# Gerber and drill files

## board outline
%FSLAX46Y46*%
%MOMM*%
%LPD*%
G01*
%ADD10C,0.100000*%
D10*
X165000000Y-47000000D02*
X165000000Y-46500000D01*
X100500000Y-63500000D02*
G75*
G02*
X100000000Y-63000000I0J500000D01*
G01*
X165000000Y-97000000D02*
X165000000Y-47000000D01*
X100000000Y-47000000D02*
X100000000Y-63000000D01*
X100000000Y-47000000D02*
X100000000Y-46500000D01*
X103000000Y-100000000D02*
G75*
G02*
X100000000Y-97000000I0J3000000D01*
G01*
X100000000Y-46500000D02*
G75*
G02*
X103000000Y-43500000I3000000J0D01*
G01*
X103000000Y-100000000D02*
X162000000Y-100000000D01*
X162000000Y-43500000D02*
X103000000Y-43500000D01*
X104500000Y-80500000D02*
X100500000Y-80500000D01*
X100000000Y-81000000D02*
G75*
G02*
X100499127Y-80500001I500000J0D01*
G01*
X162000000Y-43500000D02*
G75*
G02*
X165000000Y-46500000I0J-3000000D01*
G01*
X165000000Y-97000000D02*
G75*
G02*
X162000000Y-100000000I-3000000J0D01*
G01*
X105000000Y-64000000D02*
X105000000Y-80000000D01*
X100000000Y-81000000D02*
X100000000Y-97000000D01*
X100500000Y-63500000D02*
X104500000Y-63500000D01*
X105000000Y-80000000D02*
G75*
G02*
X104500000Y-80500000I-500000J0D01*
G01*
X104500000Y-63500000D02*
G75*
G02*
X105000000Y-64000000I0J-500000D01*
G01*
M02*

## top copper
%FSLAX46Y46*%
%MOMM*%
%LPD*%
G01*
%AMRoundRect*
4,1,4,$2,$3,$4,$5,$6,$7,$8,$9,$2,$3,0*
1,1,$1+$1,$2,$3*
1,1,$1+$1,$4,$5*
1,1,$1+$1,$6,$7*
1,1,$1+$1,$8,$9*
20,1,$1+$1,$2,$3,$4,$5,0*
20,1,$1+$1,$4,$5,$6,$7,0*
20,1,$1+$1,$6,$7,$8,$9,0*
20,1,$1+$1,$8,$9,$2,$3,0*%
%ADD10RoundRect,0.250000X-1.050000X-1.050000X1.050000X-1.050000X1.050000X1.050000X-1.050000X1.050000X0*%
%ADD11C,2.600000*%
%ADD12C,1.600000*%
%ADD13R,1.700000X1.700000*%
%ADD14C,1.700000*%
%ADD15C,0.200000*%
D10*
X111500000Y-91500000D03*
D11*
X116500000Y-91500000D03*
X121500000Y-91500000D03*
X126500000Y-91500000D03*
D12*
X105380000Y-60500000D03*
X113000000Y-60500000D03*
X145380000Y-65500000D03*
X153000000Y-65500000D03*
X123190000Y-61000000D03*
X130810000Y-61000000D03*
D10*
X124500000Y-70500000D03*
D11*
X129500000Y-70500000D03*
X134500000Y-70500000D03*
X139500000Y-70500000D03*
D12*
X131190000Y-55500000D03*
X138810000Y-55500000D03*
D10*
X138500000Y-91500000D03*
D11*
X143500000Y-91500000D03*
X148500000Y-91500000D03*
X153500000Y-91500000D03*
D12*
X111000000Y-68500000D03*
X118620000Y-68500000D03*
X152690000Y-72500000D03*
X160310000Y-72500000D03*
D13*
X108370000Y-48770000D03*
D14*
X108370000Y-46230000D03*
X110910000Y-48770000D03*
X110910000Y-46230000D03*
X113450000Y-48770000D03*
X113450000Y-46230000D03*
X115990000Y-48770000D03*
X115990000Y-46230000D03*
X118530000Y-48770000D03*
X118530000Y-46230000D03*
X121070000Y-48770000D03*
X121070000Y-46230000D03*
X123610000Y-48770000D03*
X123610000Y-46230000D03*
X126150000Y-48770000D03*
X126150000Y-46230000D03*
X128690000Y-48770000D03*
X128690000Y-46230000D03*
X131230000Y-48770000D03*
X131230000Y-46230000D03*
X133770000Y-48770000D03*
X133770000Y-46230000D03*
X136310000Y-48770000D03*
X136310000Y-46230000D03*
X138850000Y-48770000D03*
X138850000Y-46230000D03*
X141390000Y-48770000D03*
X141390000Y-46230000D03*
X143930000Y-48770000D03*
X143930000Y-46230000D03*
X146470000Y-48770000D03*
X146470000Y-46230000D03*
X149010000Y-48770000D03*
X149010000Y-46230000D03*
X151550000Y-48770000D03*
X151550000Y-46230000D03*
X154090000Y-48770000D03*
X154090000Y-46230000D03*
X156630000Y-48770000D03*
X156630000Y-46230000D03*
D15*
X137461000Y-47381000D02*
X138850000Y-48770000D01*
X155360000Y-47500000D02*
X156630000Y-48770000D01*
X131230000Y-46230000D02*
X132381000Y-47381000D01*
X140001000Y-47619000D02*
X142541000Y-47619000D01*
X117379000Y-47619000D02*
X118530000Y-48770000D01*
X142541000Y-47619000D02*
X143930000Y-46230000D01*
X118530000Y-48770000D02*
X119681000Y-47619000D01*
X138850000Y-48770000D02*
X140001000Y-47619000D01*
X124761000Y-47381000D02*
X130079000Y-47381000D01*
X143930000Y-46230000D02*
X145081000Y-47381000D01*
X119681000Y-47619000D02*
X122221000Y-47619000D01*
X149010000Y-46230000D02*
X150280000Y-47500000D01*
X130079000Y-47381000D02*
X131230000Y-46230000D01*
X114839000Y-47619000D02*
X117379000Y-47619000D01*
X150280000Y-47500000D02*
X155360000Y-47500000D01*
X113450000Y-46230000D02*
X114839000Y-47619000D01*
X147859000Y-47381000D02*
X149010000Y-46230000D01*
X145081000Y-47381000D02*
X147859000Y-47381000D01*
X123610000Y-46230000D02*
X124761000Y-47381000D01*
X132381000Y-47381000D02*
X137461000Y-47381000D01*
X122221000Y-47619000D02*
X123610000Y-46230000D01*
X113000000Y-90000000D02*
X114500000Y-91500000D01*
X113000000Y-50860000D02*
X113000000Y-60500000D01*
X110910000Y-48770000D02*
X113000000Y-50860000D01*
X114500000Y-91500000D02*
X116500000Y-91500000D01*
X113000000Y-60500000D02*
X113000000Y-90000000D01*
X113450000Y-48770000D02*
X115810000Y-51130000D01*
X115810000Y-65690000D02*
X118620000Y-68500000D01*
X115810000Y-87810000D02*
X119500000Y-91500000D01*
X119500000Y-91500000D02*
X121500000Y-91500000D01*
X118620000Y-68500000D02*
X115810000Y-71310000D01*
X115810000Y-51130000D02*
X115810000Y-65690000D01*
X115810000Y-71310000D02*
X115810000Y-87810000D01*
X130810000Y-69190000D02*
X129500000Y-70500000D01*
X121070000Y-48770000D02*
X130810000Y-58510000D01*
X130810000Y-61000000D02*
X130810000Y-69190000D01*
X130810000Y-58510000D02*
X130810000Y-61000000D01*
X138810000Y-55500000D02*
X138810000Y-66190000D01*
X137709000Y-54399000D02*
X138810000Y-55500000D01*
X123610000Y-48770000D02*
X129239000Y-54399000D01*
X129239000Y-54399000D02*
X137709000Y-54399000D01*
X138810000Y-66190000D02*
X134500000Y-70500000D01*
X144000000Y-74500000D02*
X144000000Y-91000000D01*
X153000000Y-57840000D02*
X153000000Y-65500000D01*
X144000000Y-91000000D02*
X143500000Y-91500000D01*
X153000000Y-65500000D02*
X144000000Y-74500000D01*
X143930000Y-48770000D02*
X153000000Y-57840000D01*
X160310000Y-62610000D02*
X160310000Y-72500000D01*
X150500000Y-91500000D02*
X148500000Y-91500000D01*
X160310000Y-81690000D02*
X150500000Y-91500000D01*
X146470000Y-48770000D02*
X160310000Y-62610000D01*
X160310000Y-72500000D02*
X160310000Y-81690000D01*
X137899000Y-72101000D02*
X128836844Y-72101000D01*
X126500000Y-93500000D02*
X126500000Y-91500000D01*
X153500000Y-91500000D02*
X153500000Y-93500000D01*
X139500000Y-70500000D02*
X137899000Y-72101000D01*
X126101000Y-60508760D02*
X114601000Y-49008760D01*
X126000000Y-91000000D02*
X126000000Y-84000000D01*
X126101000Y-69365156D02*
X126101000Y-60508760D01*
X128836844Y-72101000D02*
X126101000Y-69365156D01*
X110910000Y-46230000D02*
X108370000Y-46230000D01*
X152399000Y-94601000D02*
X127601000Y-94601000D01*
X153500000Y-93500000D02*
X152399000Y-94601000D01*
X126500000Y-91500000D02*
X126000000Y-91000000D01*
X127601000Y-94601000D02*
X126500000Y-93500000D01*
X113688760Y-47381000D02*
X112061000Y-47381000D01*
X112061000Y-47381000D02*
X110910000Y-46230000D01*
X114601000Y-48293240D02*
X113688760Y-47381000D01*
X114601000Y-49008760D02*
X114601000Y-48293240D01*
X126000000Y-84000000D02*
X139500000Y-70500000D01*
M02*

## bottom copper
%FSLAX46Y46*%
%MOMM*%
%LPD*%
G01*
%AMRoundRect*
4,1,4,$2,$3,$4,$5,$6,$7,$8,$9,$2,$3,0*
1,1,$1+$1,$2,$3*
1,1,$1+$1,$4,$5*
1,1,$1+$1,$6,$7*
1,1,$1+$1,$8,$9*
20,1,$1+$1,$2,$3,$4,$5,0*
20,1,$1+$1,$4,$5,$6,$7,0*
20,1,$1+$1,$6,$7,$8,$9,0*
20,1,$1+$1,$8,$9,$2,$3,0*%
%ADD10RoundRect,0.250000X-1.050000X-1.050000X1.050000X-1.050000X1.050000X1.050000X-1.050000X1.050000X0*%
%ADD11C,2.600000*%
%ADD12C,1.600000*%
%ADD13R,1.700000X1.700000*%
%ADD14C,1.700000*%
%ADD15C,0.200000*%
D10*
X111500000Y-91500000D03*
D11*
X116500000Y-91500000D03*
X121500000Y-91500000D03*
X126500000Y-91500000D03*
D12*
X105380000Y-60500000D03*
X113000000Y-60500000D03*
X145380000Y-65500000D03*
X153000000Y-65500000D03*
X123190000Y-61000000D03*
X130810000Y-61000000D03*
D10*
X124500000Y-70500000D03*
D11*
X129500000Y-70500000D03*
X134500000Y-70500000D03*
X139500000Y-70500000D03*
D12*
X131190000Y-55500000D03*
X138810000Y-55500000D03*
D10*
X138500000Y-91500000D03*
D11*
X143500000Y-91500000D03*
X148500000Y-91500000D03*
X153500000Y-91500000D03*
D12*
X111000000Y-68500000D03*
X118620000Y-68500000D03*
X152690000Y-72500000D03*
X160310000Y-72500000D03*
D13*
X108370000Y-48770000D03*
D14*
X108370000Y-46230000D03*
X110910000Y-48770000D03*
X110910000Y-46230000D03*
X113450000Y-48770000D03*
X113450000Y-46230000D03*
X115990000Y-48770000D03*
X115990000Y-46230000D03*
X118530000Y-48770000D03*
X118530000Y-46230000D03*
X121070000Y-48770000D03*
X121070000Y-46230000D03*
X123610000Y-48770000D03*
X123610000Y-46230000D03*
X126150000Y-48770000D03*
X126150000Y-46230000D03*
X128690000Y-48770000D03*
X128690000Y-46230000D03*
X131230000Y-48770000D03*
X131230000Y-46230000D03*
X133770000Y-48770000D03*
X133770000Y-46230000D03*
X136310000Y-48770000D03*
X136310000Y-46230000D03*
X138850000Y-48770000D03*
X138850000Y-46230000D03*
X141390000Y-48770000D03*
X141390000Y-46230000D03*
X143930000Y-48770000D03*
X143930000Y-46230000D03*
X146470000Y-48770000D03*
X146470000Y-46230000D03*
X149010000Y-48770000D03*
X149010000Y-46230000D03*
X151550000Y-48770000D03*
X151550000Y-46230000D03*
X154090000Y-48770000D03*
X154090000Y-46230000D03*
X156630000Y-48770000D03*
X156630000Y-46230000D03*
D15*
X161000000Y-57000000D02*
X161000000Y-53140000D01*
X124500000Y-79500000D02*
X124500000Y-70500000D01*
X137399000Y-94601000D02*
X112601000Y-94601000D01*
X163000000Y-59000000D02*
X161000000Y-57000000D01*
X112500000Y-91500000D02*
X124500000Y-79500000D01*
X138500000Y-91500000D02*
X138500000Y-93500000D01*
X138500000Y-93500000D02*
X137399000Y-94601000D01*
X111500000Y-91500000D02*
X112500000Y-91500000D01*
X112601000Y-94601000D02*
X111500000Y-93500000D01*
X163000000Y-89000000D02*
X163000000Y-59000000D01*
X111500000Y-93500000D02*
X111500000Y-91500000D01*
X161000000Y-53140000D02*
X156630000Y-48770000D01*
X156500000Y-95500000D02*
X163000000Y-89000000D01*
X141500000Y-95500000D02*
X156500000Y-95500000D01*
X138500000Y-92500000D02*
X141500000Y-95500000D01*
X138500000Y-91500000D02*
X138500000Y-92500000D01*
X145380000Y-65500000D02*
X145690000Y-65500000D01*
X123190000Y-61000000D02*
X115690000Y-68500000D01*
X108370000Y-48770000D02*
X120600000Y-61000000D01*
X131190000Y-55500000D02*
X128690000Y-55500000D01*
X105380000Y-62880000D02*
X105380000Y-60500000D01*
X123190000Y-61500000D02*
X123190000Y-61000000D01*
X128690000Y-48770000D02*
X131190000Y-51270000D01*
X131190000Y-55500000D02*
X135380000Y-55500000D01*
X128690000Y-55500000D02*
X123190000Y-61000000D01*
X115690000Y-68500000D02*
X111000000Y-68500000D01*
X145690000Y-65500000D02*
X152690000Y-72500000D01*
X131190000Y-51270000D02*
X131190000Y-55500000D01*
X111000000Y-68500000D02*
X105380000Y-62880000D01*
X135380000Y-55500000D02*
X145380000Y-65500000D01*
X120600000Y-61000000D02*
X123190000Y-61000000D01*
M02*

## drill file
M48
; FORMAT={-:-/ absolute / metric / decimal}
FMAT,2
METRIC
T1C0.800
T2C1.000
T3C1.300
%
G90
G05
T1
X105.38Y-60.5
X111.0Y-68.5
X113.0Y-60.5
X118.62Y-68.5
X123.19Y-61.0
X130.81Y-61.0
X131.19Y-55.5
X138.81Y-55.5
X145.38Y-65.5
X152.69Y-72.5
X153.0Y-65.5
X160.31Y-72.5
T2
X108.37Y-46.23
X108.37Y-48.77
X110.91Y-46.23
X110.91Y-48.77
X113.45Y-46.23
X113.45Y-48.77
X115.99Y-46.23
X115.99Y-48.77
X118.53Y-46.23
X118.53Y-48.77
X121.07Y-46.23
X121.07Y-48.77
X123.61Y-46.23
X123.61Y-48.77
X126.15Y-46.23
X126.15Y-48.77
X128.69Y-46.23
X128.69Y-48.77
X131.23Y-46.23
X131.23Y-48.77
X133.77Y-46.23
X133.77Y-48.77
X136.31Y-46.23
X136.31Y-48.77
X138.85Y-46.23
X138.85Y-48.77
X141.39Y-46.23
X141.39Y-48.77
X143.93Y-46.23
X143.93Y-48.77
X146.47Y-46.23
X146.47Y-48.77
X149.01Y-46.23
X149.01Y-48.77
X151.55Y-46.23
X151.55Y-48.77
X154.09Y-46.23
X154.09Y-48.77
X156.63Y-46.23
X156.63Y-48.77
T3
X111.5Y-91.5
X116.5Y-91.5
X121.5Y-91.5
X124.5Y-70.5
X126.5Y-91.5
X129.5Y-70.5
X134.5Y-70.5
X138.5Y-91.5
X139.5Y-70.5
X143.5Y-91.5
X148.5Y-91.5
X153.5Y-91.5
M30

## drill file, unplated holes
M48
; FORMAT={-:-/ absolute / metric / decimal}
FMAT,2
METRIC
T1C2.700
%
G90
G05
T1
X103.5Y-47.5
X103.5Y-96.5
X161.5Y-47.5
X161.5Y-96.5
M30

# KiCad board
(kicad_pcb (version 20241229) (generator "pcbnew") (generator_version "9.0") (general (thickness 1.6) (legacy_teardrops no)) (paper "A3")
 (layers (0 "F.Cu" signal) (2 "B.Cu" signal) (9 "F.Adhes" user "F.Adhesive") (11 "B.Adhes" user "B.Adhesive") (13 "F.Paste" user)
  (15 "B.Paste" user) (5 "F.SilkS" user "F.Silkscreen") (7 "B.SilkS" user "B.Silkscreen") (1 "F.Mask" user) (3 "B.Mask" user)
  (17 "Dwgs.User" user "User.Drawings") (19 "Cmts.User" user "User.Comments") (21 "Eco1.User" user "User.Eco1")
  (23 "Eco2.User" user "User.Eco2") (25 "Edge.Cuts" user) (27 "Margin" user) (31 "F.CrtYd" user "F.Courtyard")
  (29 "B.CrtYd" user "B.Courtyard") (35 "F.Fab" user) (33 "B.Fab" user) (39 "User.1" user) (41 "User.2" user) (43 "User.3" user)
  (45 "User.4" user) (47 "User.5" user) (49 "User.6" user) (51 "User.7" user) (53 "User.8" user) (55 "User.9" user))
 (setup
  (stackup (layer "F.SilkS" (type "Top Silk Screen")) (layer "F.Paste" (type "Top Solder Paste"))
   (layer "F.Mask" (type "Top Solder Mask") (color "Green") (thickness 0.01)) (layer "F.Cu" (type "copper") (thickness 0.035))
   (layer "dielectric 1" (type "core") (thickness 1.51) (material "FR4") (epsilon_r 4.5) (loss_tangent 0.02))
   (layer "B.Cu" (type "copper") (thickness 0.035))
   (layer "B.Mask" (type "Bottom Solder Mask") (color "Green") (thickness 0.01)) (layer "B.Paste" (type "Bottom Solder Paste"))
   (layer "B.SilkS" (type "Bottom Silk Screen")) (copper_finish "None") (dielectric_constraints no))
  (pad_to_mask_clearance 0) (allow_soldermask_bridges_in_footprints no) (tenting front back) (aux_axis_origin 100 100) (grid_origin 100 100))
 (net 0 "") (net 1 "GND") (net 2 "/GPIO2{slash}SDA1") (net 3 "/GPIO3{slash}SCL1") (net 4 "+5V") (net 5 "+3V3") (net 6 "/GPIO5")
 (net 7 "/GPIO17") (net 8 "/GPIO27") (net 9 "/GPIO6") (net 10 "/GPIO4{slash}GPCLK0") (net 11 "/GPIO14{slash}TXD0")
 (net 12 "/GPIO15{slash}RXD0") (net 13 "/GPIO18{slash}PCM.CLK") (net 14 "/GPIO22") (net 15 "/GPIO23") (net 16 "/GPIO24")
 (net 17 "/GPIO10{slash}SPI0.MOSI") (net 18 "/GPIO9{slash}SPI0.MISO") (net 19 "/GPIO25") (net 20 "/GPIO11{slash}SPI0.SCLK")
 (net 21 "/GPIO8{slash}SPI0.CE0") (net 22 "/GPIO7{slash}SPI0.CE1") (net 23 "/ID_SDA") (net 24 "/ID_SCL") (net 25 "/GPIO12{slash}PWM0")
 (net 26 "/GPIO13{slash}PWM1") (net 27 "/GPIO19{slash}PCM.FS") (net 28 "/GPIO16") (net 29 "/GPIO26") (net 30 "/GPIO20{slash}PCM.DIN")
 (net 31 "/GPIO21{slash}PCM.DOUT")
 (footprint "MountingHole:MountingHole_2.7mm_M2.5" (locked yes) (layer "F.Cu") (at 161.5 47.5)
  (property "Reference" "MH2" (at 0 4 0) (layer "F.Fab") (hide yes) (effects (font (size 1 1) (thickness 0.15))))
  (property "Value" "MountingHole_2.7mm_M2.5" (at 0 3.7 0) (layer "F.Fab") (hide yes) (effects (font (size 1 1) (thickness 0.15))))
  (pad "" np_thru_hole circle (at 0 0) (size 2.7 2.7) (drill 2.7) (layers "*.Cu" "*.Mask")))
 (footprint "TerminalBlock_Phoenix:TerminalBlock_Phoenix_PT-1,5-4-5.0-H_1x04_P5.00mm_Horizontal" (layer "F.Cu") (at 111.5 91.5)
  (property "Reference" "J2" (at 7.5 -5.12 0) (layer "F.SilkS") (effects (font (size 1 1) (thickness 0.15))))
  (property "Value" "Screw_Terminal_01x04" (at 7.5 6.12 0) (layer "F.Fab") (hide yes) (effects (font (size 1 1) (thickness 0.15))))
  (pad "1" thru_hole roundrect (at 0 0) (size 2.6 2.6) (drill 1.3) (layers "*.Cu" "*.Mask") (remove_unused_layers no)
   (roundrect_rratio 0.096154) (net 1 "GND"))
  (pad "2" thru_hole circle (at 5 0) (size 2.6 2.6) (drill 1.3) (layers "*.Cu" "*.Mask") (remove_unused_layers no)
   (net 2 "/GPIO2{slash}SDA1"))
  (pad "3" thru_hole circle (at 10 0) (size 2.6 2.6) (drill 1.3) (layers "*.Cu" "*.Mask") (remove_unused_layers no)
   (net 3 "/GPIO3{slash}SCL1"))
  (pad "4" thru_hole circle (at 15 0) (size 2.6 2.6) (drill 1.3) (layers "*.Cu" "*.Mask") (remove_unused_layers no) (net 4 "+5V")))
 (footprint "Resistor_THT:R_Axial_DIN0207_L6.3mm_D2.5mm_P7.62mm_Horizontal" (layer "F.Cu") (at 105.38 60.5)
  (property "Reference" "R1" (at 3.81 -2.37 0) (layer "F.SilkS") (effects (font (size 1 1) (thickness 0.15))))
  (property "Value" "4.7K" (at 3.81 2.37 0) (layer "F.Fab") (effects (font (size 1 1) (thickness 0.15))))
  (pad "1" thru_hole circle (at 0 0) (size 1.6 1.6) (drill 0.8) (layers "*.Cu" "*.Mask") (remove_unused_layers no) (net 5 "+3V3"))
  (pad "2" thru_hole circle (at 7.62 0) (size 1.6 1.6) (drill 0.8) (layers "*.Cu" "*.Mask") (remove_unused_layers no)
   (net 2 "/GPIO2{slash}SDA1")))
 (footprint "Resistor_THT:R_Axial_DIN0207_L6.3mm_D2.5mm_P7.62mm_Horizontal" (layer "F.Cu") (at 145.38 65.5)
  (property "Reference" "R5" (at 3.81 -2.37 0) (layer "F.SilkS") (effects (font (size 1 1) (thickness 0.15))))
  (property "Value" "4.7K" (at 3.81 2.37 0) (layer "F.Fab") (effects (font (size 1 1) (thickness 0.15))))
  (pad "1" thru_hole circle (at 0 0) (size 1.6 1.6) (drill 0.8) (layers "*.Cu" "*.Mask") (remove_unused_layers no) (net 5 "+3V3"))
  (pad "2" thru_hole circle (at 7.62 0) (size 1.6 1.6) (drill 0.8) (layers "*.Cu" "*.Mask") (remove_unused_layers no) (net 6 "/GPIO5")))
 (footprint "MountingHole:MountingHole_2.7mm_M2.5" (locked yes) (layer "F.Cu") (at 103.5 96.5)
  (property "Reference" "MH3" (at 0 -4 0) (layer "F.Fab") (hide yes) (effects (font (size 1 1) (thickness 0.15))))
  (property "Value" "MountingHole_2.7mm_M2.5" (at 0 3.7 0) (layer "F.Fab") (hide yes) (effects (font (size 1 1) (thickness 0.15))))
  (pad "" np_thru_hole circle (at 0 0) (size 2.7 2.7) (drill 2.7) (layers "*.Cu" "*.Mask")))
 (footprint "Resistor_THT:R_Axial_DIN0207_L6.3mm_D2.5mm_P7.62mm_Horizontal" (layer "F.Cu") (at 123.19 61)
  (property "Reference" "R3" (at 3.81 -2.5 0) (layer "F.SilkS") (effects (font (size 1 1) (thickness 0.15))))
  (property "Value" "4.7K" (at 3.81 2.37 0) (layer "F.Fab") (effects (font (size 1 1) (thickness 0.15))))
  (pad "1" thru_hole circle (at 0 0) (size 1.6 1.6) (drill 0.8) (layers "*.Cu" "*.Mask") (remove_unused_layers no) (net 5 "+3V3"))
  (pad "2" thru_hole circle (at 7.62 0) (size 1.6 1.6) (drill 0.8) (layers "*.Cu" "*.Mask") (remove_unused_layers no) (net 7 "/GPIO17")))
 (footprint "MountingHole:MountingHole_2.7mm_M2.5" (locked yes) (layer "F.Cu") (at 103.5 47.5)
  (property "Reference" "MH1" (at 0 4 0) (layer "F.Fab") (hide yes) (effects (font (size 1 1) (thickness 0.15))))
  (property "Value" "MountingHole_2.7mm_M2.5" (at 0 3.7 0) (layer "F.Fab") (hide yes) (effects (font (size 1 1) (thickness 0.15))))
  (pad "" np_thru_hole circle (at 0 0) (size 2.7 2.7) (drill 2.7) (layers "*.Cu" "*.Mask")))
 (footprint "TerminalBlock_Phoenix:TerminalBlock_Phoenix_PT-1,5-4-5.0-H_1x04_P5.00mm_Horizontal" (layer "F.Cu") (at 124.5 70.5)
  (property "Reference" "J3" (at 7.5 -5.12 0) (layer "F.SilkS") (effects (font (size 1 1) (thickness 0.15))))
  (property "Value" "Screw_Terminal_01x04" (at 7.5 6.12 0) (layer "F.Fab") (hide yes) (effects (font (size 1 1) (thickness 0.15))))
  (pad "1" thru_hole roundrect (at 0 0) (size 2.6 2.6) (drill 1.3) (layers "*.Cu" "*.Mask") (remove_unused_layers no)
   (roundrect_rratio 0.096154) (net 1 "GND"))
  (pad "2" thru_hole circle (at 5 0) (size 2.6 2.6) (drill 1.3) (layers "*.Cu" "*.Mask") (remove_unused_layers no) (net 7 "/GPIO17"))
  (pad "3" thru_hole circle (at 10 0) (size 2.6 2.6) (drill 1.3) (layers "*.Cu" "*.Mask") (remove_unused_layers no) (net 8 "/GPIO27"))
  (pad "4" thru_hole circle (at 15 0) (size 2.6 2.6) (drill 1.3) (layers "*.Cu" "*.Mask") (remove_unused_layers no) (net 4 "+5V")))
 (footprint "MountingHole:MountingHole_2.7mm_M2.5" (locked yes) (layer "F.Cu") (at 161.5 96.5)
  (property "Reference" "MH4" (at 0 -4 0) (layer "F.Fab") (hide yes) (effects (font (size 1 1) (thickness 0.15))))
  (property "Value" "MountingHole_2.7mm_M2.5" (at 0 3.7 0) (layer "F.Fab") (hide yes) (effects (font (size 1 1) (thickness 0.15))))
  (pad "" np_thru_hole circle (at 0 0) (size 2.7 2.7) (drill 2.7) (layers "*.Cu" "*.Mask")))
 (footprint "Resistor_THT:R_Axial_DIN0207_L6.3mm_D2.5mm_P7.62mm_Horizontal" (layer "F.Cu") (at 131.19 55.5)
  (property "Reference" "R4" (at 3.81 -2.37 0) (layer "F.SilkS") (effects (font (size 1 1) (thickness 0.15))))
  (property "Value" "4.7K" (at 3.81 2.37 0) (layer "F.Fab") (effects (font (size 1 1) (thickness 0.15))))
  (pad "1" thru_hole circle (at 0 0) (size 1.6 1.6) (drill 0.8) (layers "*.Cu" "*.Mask") (remove_unused_layers no) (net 5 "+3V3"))
  (pad "2" thru_hole circle (at 7.62 0) (size 1.6 1.6) (drill 0.8) (layers "*.Cu" "*.Mask") (remove_unused_layers no) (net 8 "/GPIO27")))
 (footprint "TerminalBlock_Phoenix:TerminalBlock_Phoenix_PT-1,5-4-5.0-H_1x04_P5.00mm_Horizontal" (layer "F.Cu") (at 138.5 91.5)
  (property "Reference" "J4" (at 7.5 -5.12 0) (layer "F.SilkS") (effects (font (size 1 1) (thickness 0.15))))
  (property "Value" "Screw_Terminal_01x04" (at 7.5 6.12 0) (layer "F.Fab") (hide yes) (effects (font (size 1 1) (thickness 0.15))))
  (pad "1" thru_hole roundrect (at 0 0) (size 2.6 2.6) (drill 1.3) (layers "*.Cu" "*.Mask") (remove_unused_layers no)
   (roundrect_rratio 0.096154) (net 1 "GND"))
  (pad "2" thru_hole circle (at 5 0) (size 2.6 2.6) (drill 1.3) (layers "*.Cu" "*.Mask") (remove_unused_layers no) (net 6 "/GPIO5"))
  (pad "3" thru_hole circle (at 10 0) (size 2.6 2.6) (drill 1.3) (layers "*.Cu" "*.Mask") (remove_unused_layers no) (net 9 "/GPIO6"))
  (pad "4" thru_hole circle (at 15 0) (size 2.6 2.6) (drill 1.3) (layers "*.Cu" "*.Mask") (remove_unused_layers no) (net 4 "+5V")))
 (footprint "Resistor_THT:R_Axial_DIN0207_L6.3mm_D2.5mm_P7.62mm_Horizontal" (layer "F.Cu") (at 111 68.5)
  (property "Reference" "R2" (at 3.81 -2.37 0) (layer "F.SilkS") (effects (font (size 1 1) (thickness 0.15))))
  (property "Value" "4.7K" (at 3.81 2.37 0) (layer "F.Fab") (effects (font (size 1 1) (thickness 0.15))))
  (pad "1" thru_hole circle (at 0 0) (size 1.6 1.6) (drill 0.8) (layers "*.Cu" "*.Mask") (remove_unused_layers no) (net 5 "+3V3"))
  (pad "2" thru_hole circle (at 7.62 0) (size 1.6 1.6) (drill 0.8) (layers "*.Cu" "*.Mask") (remove_unused_layers no)
   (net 3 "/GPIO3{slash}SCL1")))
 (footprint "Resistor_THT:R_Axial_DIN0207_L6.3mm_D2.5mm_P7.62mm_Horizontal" (layer "F.Cu") (at 152.69 72.5)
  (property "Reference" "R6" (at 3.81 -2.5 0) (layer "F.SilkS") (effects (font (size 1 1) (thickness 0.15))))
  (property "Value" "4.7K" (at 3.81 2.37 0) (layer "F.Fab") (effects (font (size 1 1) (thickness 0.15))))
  (pad "1" thru_hole circle (at 0 0) (size 1.6 1.6) (drill 0.8) (layers "*.Cu" "*.Mask") (remove_unused_layers no) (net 5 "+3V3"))
  (pad "2" thru_hole circle (at 7.62 0) (size 1.6 1.6) (drill 0.8) (layers "*.Cu" "*.Mask") (remove_unused_layers no) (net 9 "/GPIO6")))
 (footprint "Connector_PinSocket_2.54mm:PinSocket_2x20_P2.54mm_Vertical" (layer "B.Cu") (at 108.37 48.77 -90)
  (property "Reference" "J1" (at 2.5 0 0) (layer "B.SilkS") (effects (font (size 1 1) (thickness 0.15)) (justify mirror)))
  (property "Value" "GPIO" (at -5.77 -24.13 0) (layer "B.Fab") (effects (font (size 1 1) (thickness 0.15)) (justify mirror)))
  (pad "1" thru_hole rect (at 0 0 270) (size 1.7 1.7) (drill 1) (layers "*.Cu" "*.Mask") (remove_unused_layers no) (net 5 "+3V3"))
  (pad "2" thru_hole circle (at -2.54 0 270) (size 1.7 1.7) (drill 1) (layers "*.Cu" "*.Mask") (remove_unused_layers no) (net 4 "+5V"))
  (pad "3" thru_hole circle (at 0 -2.54 270) (size 1.7 1.7) (drill 1) (layers "*.Cu" "*.Mask") (remove_unused_layers no)
   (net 2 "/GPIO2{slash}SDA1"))
  (pad "4" thru_hole circle (at -2.54 -2.54 270) (size 1.7 1.7) (drill 1) (layers "*.Cu" "*.Mask") (remove_unused_layers no) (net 4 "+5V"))
  (pad "5" thru_hole circle (at 0 -5.08 270) (size 1.7 1.7) (drill 1) (layers "*.Cu" "*.Mask") (remove_unused_layers no)
   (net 3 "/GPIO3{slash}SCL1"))
  (pad "6" thru_hole circle (at -2.54 -5.08 270) (size 1.7 1.7) (drill 1) (layers "*.Cu" "*.Mask") (remove_unused_layers no) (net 1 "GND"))
  (pad "7" thru_hole circle (at 0 -7.62 270) (size 1.7 1.7) (drill 1) (layers "*.Cu" "*.Mask") (remove_unused_layers no)
   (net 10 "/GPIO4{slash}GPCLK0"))
  (pad "8" thru_hole circle (at -2.54 -7.62 270) (size 1.7 1.7) (drill 1) (layers "*.Cu" "*.Mask") (remove_unused_layers no)
   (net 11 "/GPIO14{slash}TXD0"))
  (pad "9" thru_hole circle (at 0 -10.16 270) (size 1.7 1.7) (drill 1) (layers "*.Cu" "*.Mask") (remove_unused_layers no) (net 1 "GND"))
  (pad "10" thru_hole circle (at -2.54 -10.16 270) (size 1.7 1.7) (drill 1) (layers "*.Cu" "*.Mask") (remove_unused_layers no)
   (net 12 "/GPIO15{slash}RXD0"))
  (pad "11" thru_hole circle (at 0 -12.7 270) (size 1.7 1.7) (drill 1) (layers "*.Cu" "*.Mask") (remove_unused_layers no) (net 7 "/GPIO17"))
  (pad "12" thru_hole circle (at -2.54 -12.7 270) (size 1.7 1.7) (drill 1) (layers "*.Cu" "*.Mask") (remove_unused_layers no)
   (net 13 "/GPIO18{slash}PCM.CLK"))
  (pad "13" thru_hole circle (at 0 -15.24 270) (size 1.7 1.7) (drill 1) (layers "*.Cu" "*.Mask") (remove_unused_layers no) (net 8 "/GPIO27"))
  (pad "14" thru_hole circle (at -2.54 -15.24 270) (size 1.7 1.7) (drill 1) (layers "*.Cu" "*.Mask") (remove_unused_layers no) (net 1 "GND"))
  (pad "15" thru_hole circle (at 0 -17.78 270) (size 1.7 1.7) (drill 1) (layers "*.Cu" "*.Mask") (remove_unused_layers no)
   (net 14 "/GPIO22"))
  (pad "16" thru_hole circle (at -2.54 -17.78 270) (size 1.7 1.7) (drill 1) (layers "*.Cu" "*.Mask") (remove_unused_layers no)
   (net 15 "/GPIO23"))
  (pad "17" thru_hole circle (at 0 -20.32 270) (size 1.7 1.7) (drill 1) (layers "*.Cu" "*.Mask") (remove_unused_layers no) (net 5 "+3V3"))
  (pad "18" thru_hole circle (at -2.54 -20.32 270) (size 1.7 1.7) (drill 1) (layers "*.Cu" "*.Mask") (remove_unused_layers no)
   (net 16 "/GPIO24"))
  (pad "19" thru_hole circle (at 0 -22.86 270) (size 1.7 1.7) (drill 1) (layers "*.Cu" "*.Mask") (remove_unused_layers no)
   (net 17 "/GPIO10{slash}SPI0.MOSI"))
  (pad "20" thru_hole circle (at -2.54 -22.86 270) (size 1.7 1.7) (drill 1) (layers "*.Cu" "*.Mask") (remove_unused_layers no) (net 1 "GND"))
  (pad "21" thru_hole circle (at 0 -25.4 270) (size 1.7 1.7) (drill 1) (layers "*.Cu" "*.Mask") (remove_unused_layers no)
   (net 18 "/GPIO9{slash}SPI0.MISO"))
  (pad "22" thru_hole circle (at -2.54 -25.4 270) (size 1.7 1.7) (drill 1) (layers "*.Cu" "*.Mask") (remove_unused_layers no)
   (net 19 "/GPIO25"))
  (pad "23" thru_hole circle (at 0 -27.94 270) (size 1.7 1.7) (drill 1) (layers "*.Cu" "*.Mask") (remove_unused_layers no)
   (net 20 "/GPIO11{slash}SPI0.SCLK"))
  (pad "24" thru_hole circle (at -2.54 -27.94 270) (size 1.7 1.7) (drill 1) (layers "*.Cu" "*.Mask") (remove_unused_layers no)
   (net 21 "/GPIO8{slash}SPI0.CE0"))
  (pad "25" thru_hole circle (at 0 -30.48 270) (size 1.7 1.7) (drill 1) (layers "*.Cu" "*.Mask") (remove_unused_layers no) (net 1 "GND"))
  (pad "26" thru_hole circle (at -2.54 -30.48 270) (size 1.7 1.7) (drill 1) (layers "*.Cu" "*.Mask") (remove_unused_layers no)
   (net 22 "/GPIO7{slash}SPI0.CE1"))
  (pad "27" thru_hole circle (at 0 -33.02 270) (size 1.7 1.7) (drill 1) (layers "*.Cu" "*.Mask") (remove_unused_layers no)
   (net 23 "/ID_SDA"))
  (pad "28" thru_hole circle (at -2.54 -33.02 270) (size 1.7 1.7) (drill 1) (layers "*.Cu" "*.Mask") (remove_unused_layers no)
   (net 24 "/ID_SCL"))
  (pad "29" thru_hole circle (at 0 -35.56 270) (size 1.7 1.7) (drill 1) (layers "*.Cu" "*.Mask") (remove_unused_layers no) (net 6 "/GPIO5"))
  (pad "30" thru_hole circle (at -2.54 -35.56 270) (size 1.7 1.7) (drill 1) (layers "*.Cu" "*.Mask") (remove_unused_layers no) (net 1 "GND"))
  (pad "31" thru_hole circle (at 0 -38.1 270) (size 1.7 1.7) (drill 1) (layers "*.Cu" "*.Mask") (remove_unused_layers no) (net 9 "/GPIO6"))
  (pad "32" thru_hole circle (at -2.54 -38.1 270) (size 1.7 1.7) (drill 1) (layers "*.Cu" "*.Mask") (remove_unused_layers no)
   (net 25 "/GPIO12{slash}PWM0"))
  (pad "33" thru_hole circle (at 0 -40.64 270) (size 1.7 1.7) (drill 1) (layers "*.Cu" "*.Mask") (remove_unused_layers no)
   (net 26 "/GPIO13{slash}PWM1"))
  (pad "34" thru_hole circle (at -2.54 -40.64 270) (size 1.7 1.7) (drill 1) (layers "*.Cu" "*.Mask") (remove_unused_layers no) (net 1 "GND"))
  (pad "35" thru_hole circle (at 0 -43.18 270) (size 1.7 1.7) (drill 1) (layers "*.Cu" "*.Mask") (remove_unused_layers no)
   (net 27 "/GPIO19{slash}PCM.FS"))
  (pad "36" thru_hole circle (at -2.54 -43.18 270) (size 1.7 1.7) (drill 1) (layers "*.Cu" "*.Mask") (remove_unused_layers no)
   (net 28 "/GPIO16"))
  (pad "37" thru_hole circle (at 0 -45.72 270) (size 1.7 1.7) (drill 1) (layers "*.Cu" "*.Mask") (remove_unused_layers no)
   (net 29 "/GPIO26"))
  (pad "38" thru_hole circle (at -2.54 -45.72 270) (size 1.7 1.7) (drill 1) (layers "*.Cu" "*.Mask") (remove_unused_layers no)
   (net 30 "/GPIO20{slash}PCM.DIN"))
  (pad "39" thru_hole circle (at 0 -48.26 270) (size 1.7 1.7) (drill 1) (layers "*.Cu" "*.Mask") (remove_unused_layers no) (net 1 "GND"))
  (pad "40" thru_hole circle (at -2.54 -48.26 270) (size 1.7 1.7) (drill 1) (layers "*.Cu" "*.Mask") (remove_unused_layers no)
   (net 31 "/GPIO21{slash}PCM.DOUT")))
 (gr_line (start 165 47) (end 165 46.5) (stroke (width 0.1) (type solid)) (layer "Edge.Cuts"))
 (gr_arc (start 100.5 63.5) (mid 100.146447 63.353553) (end 100 63) (stroke (width 0.1) (type solid)) (layer "Edge.Cuts"))
 (gr_line (start 165 97) (end 165 47) (stroke (width 0.1) (type solid)) (layer "Edge.Cuts"))
 (gr_line (start 100 47) (end 100 63) (stroke (width 0.1) (type solid)) (layer "Edge.Cuts"))
 (gr_line (start 100 47) (end 100 46.5) (stroke (width 0.1) (type solid)) (layer "Edge.Cuts"))
 (gr_arc (start 103 100) (mid 100.87868 99.12132) (end 100 97) (stroke (width 0.1) (type solid)) (layer "Edge.Cuts"))
 (gr_arc (start 100 46.5) (mid 100.87868 44.37868) (end 103 43.5) (stroke (width 0.1) (type solid)) (layer "Edge.Cuts"))
 (gr_line (start 103 100) (end 162 100) (stroke (width 0.1) (type solid)) (layer "Edge.Cuts"))
 (gr_line (start 162 43.5) (end 103 43.5) (stroke (width 0.1) (type solid)) (layer "Edge.Cuts"))
 (gr_line (start 104.5 80.5) (end 100.5 80.5) (stroke (width 0.1) (type solid)) (layer "Edge.Cuts"))
 (gr_arc (start 100 81) (mid 100.146138 80.646755) (end 100.499127 80.500001) (stroke (width 0.1) (type solid)) (layer "Edge.Cuts"))
 (gr_arc (start 162 43.5) (mid 164.12132 44.37868) (end 165 46.5) (stroke (width 0.1) (type solid)) (layer "Edge.Cuts"))
 (gr_arc (start 165 97) (mid 164.12132 99.12132) (end 162 100) (stroke (width 0.1) (type solid)) (layer "Edge.Cuts"))
 (gr_line (start 105 64) (end 105 80) (stroke (width 0.1) (type solid)) (layer "Edge.Cuts"))
 (gr_line (start 100 81) (end 100 97) (stroke (width 0.1) (type solid)) (layer "Edge.Cuts"))
 (gr_line (start 100.5 63.5) (end 104.5 63.5) (stroke (width 0.1) (type solid)) (layer "Edge.Cuts"))
 (gr_arc (start 105 80) (mid 104.853553 80.353553) (end 104.5 80.5) (stroke (width 0.1) (type solid)) (layer "Edge.Cuts"))
 (gr_arc (start 104.5 63.5) (mid 104.853553 63.646447) (end 105 64) (stroke (width 0.1) (type solid)) (layer "Edge.Cuts"))
 (segment (start 137.461 47.381) (end 138.85 48.77) (width 0.2) (layer "F.Cu") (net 1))
 (segment (start 155.36 47.5) (end 156.63 48.77) (width 0.2) (layer "F.Cu") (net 1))
 (segment (start 131.23 46.23) (end 132.381 47.381) (width 0.2) (layer "F.Cu") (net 1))
 (segment (start 140.001 47.619) (end 142.541 47.619) (width 0.2) (layer "F.Cu") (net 1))
 (segment (start 117.379 47.619) (end 118.53 48.77) (width 0.2) (layer "F.Cu") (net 1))
 (segment (start 142.541 47.619) (end 143.93 46.23) (width 0.2) (layer "F.Cu") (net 1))
 (segment (start 118.53 48.77) (end 119.681 47.619) (width 0.2) (layer "F.Cu") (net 1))
 (segment (start 138.85 48.77) (end 140.001 47.619) (width 0.2) (layer "F.Cu") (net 1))
 (segment (start 124.761 47.381) (end 130.079 47.381) (width 0.2) (layer "F.Cu") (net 1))
 (segment (start 143.93 46.23) (end 145.081 47.381) (width 0.2) (layer "F.Cu") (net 1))
 (segment (start 119.681 47.619) (end 122.221 47.619) (width 0.2) (layer "F.Cu") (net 1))
 (segment (start 149.01 46.23) (end 150.28 47.5) (width 0.2) (layer "F.Cu") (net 1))
 (segment (start 130.079 47.381) (end 131.23 46.23) (width 0.2) (layer "F.Cu") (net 1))
 (segment (start 114.839 47.619) (end 117.379 47.619) (width 0.2) (layer "F.Cu") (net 1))
 (segment (start 150.28 47.5) (end 155.36 47.5) (width 0.2) (layer "F.Cu") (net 1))
 (segment (start 113.45 46.23) (end 114.839 47.619) (width 0.2) (layer "F.Cu") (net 1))
 (segment (start 147.859 47.381) (end 149.01 46.23) (width 0.2) (layer "F.Cu") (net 1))
 (segment (start 145.081 47.381) (end 147.859 47.381) (width 0.2) (layer "F.Cu") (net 1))
 (segment (start 123.61 46.23) (end 124.761 47.381) (width 0.2) (layer "F.Cu") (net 1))
 (segment (start 132.381 47.381) (end 137.461 47.381) (width 0.2) (layer "F.Cu") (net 1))
 (segment (start 122.221 47.619) (end 123.61 46.23) (width 0.2) (layer "F.Cu") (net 1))
 (segment (start 161 57) (end 161 53.14) (width 0.2) (layer "B.Cu") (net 1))
 (segment (start 124.5 79.5) (end 124.5 70.5) (width 0.2) (layer "B.Cu") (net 1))
 (segment (start 137.399 94.601) (end 112.601 94.601) (width 0.2) (layer "B.Cu") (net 1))
 (segment (start 163 59) (end 161 57) (width 0.2) (layer "B.Cu") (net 1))
 (segment (start 112.5 91.5) (end 124.5 79.5) (width 0.2) (layer "B.Cu") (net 1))
 (segment (start 138.5 91.5) (end 138.5 93.5) (width 0.2) (layer "B.Cu") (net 1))
 (segment (start 138.5 93.5) (end 137.399 94.601) (width 0.2) (layer "B.Cu") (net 1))
 (segment (start 111.5 91.5) (end 112.5 91.5) (width 0.2) (layer "B.Cu") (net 1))
 (segment (start 112.601 94.601) (end 111.5 93.5) (width 0.2) (layer "B.Cu") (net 1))
 (segment (start 163 89) (end 163 59) (width 0.2) (layer "B.Cu") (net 1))
 (segment (start 111.5 93.5) (end 111.5 91.5) (width 0.2) (layer "B.Cu") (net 1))
 (segment (start 161 53.14) (end 156.63 48.77) (width 0.2) (layer "B.Cu") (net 1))
 (segment (start 156.5 95.5) (end 163 89) (width 0.2) (layer "B.Cu") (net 1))
 (segment (start 141.5 95.5) (end 156.5 95.5) (width 0.2) (layer "B.Cu") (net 1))
 (segment (start 138.5 92.5) (end 141.5 95.5) (width 0.2) (layer "B.Cu") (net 1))
 (segment (start 138.5 91.5) (end 138.5 92.5) (width 0.2) (layer "B.Cu") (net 1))
 (segment (start 113 90) (end 114.5 91.5) (width 0.2) (layer "F.Cu") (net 2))
 (segment (start 113 50.86) (end 113 60.5) (width 0.2) (layer "F.Cu") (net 2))
 (segment (start 110.91 48.77) (end 113 50.86) (width 0.2) (layer "F.Cu") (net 2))
 (segment (start 114.5 91.5) (end 116.5 91.5) (width 0.2) (layer "F.Cu") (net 2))
 (segment (start 113 60.5) (end 113 90) (width 0.2) (layer "F.Cu") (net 2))
 (segment (start 113.45 48.77) (end 115.81 51.13) (width 0.2) (layer "F.Cu") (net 3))
 (segment (start 115.81 65.69) (end 118.62 68.5) (width 0.2) (layer "F.Cu") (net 3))
 (segment (start 115.81 87.81) (end 119.5 91.5) (width 0.2) (layer "F.Cu") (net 3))
 (segment (start 119.5 91.5) (end 121.5 91.5) (width 0.2) (layer "F.Cu") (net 3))
 (segment (start 118.62 68.5) (end 115.81 71.31) (width 0.2) (layer "F.Cu") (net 3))
 (segment (start 115.81 51.13) (end 115.81 65.69) (width 0.2) (layer "F.Cu") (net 3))
 (segment (start 115.81 71.31) (end 115.81 87.81) (width 0.2) (layer "F.Cu") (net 3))
 (segment (start 130.81 69.19) (end 129.5 70.5) (width 0.2) (layer "F.Cu") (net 7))
 (segment (start 121.07 48.77) (end 130.81 58.51) (width 0.2) (layer "F.Cu") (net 7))
 (segment (start 130.81 61) (end 130.81 69.19) (width 0.2) (layer "F.Cu") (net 7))
 (segment (start 130.81 58.51) (end 130.81 61) (width 0.2) (layer "F.Cu") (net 7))
 (segment (start 138.81 55.5) (end 138.81 66.19) (width 0.2) (layer "F.Cu") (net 8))
 (segment (start 137.709 54.399) (end 138.81 55.5) (width 0.2) (layer "F.Cu") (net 8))
 (segment (start 123.61 48.77) (end 129.239 54.399) (width 0.2) (layer "F.Cu") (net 8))
 (segment (start 129.239 54.399) (end 137.709 54.399) (width 0.2) (layer "F.Cu") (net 8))
 (segment (start 138.81 66.19) (end 134.5 70.5) (width 0.2) (layer "F.Cu") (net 8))
 (segment (start 144 74.5) (end 144 91) (width 0.2) (layer "F.Cu") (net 6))
 (segment (start 153 57.84) (end 153 65.5) (width 0.2) (layer "F.Cu") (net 6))
 (segment (start 144 91) (end 143.5 91.5) (width 0.2) (layer "F.Cu") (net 6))
 (segment (start 153 65.5) (end 144 74.5) (width 0.2) (layer "F.Cu") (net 6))
 (segment (start 143.93 48.77) (end 153 57.84) (width 0.2) (layer "F.Cu") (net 6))
 (segment (start 160.31 62.61) (end 160.31 72.5) (width 0.2) (layer "F.Cu") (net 9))
 (segment (start 150.5 91.5) (end 148.5 91.5) (width 0.2) (layer "F.Cu") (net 9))
 (segment (start 160.31 81.69) (end 150.5 91.5) (width 0.2) (layer "F.Cu") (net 9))
 (segment (start 146.47 48.77) (end 160.31 62.61) (width 0.2) (layer "F.Cu") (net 9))
 (segment (start 160.31 72.5) (end 160.31 81.69) (width 0.2) (layer "F.Cu") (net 9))
 (segment (start 137.899 72.101) (end 128.836844 72.101) (width 0.2) (layer "F.Cu") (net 4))
 (segment (start 126.5 93.5) (end 126.5 91.5) (width 0.2) (layer "F.Cu") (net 4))
 (segment (start 153.5 91.5) (end 153.5 93.5) (width 0.2) (layer "F.Cu") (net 4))
 (segment (start 139.5 70.5) (end 137.899 72.101) (width 0.2) (layer "F.Cu") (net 4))
 (segment (start 126.101 60.50876) (end 114.601 49.00876) (width 0.2) (layer "F.Cu") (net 4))
 (segment (start 126 91) (end 126 84) (width 0.2) (layer "F.Cu") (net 4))
 (segment (start 126.101 69.365156) (end 126.101 60.50876) (width 0.2) (layer "F.Cu") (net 4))
 (segment (start 128.836844 72.101) (end 126.101 69.365156) (width 0.2) (layer "F.Cu") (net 4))
 (segment (start 110.91 46.23) (end 108.37 46.23) (width 0.2) (layer "F.Cu") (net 4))
 (segment (start 152.399 94.601) (end 127.601 94.601) (width 0.2) (layer "F.Cu") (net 4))
 (segment (start 153.5 93.5) (end 152.399 94.601) (width 0.2) (layer "F.Cu") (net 4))
 (segment (start 126.5 91.5) (end 126 91) (width 0.2) (layer "F.Cu") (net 4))
 (segment (start 127.601 94.601) (end 126.5 93.5) (width 0.2) (layer "F.Cu") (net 4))
 (segment (start 113.68876 47.381) (end 112.061 47.381) (width 0.2) (layer "F.Cu") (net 4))
 (segment (start 112.061 47.381) (end 110.91 46.23) (width 0.2) (layer "F.Cu") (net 4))
 (segment (start 114.601 48.29324) (end 113.68876 47.381) (width 0.2) (layer "F.Cu") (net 4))
 (segment (start 114.601 49.00876) (end 114.601 48.29324) (width 0.2) (layer "F.Cu") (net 4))
 (segment (start 126 84) (end 139.5 70.5) (width 0.2) (layer "F.Cu") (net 4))
 (segment (start 145.38 65.5) (end 145.69 65.5) (width 0.2) (layer "B.Cu") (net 5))
 (segment (start 123.19 61) (end 115.69 68.5) (width 0.2) (layer "B.Cu") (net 5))
 (segment (start 108.37 48.77) (end 120.6 61) (width 0.2) (layer "B.Cu") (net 5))
 (segment (start 131.19 55.5) (end 128.69 55.5) (width 0.2) (layer "B.Cu") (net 5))
 (segment (start 105.38 62.88) (end 105.38 60.5) (width 0.2) (layer "B.Cu") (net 5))
 (segment (start 123.19 61.5) (end 123.19 61) (width 0.2) (layer "B.Cu") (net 5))
 (segment (start 128.69 48.77) (end 131.19 51.27) (width 0.2) (layer "B.Cu") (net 5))
 (segment (start 131.19 55.5) (end 135.38 55.5) (width 0.2) (layer "B.Cu") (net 5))
 (segment (start 128.69 55.5) (end 123.19 61) (width 0.2) (layer "B.Cu") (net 5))
 (segment (start 115.69 68.5) (end 111 68.5) (width 0.2) (layer "B.Cu") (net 5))
 (segment (start 145.69 65.5) (end 152.69 72.5) (width 0.2) (layer "B.Cu") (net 5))
 (segment (start 131.19 51.27) (end 131.19 55.5) (width 0.2) (layer "B.Cu") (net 5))
 (segment (start 111 68.5) (end 105.38 62.88) (width 0.2) (layer "B.Cu") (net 5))
 (segment (start 135.38 55.5) (end 145.38 65.5) (width 0.2) (layer "B.Cu") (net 5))
 (segment (start 120.6 61) (end 123.19 61) (width 0.2) (layer "B.Cu") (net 5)))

